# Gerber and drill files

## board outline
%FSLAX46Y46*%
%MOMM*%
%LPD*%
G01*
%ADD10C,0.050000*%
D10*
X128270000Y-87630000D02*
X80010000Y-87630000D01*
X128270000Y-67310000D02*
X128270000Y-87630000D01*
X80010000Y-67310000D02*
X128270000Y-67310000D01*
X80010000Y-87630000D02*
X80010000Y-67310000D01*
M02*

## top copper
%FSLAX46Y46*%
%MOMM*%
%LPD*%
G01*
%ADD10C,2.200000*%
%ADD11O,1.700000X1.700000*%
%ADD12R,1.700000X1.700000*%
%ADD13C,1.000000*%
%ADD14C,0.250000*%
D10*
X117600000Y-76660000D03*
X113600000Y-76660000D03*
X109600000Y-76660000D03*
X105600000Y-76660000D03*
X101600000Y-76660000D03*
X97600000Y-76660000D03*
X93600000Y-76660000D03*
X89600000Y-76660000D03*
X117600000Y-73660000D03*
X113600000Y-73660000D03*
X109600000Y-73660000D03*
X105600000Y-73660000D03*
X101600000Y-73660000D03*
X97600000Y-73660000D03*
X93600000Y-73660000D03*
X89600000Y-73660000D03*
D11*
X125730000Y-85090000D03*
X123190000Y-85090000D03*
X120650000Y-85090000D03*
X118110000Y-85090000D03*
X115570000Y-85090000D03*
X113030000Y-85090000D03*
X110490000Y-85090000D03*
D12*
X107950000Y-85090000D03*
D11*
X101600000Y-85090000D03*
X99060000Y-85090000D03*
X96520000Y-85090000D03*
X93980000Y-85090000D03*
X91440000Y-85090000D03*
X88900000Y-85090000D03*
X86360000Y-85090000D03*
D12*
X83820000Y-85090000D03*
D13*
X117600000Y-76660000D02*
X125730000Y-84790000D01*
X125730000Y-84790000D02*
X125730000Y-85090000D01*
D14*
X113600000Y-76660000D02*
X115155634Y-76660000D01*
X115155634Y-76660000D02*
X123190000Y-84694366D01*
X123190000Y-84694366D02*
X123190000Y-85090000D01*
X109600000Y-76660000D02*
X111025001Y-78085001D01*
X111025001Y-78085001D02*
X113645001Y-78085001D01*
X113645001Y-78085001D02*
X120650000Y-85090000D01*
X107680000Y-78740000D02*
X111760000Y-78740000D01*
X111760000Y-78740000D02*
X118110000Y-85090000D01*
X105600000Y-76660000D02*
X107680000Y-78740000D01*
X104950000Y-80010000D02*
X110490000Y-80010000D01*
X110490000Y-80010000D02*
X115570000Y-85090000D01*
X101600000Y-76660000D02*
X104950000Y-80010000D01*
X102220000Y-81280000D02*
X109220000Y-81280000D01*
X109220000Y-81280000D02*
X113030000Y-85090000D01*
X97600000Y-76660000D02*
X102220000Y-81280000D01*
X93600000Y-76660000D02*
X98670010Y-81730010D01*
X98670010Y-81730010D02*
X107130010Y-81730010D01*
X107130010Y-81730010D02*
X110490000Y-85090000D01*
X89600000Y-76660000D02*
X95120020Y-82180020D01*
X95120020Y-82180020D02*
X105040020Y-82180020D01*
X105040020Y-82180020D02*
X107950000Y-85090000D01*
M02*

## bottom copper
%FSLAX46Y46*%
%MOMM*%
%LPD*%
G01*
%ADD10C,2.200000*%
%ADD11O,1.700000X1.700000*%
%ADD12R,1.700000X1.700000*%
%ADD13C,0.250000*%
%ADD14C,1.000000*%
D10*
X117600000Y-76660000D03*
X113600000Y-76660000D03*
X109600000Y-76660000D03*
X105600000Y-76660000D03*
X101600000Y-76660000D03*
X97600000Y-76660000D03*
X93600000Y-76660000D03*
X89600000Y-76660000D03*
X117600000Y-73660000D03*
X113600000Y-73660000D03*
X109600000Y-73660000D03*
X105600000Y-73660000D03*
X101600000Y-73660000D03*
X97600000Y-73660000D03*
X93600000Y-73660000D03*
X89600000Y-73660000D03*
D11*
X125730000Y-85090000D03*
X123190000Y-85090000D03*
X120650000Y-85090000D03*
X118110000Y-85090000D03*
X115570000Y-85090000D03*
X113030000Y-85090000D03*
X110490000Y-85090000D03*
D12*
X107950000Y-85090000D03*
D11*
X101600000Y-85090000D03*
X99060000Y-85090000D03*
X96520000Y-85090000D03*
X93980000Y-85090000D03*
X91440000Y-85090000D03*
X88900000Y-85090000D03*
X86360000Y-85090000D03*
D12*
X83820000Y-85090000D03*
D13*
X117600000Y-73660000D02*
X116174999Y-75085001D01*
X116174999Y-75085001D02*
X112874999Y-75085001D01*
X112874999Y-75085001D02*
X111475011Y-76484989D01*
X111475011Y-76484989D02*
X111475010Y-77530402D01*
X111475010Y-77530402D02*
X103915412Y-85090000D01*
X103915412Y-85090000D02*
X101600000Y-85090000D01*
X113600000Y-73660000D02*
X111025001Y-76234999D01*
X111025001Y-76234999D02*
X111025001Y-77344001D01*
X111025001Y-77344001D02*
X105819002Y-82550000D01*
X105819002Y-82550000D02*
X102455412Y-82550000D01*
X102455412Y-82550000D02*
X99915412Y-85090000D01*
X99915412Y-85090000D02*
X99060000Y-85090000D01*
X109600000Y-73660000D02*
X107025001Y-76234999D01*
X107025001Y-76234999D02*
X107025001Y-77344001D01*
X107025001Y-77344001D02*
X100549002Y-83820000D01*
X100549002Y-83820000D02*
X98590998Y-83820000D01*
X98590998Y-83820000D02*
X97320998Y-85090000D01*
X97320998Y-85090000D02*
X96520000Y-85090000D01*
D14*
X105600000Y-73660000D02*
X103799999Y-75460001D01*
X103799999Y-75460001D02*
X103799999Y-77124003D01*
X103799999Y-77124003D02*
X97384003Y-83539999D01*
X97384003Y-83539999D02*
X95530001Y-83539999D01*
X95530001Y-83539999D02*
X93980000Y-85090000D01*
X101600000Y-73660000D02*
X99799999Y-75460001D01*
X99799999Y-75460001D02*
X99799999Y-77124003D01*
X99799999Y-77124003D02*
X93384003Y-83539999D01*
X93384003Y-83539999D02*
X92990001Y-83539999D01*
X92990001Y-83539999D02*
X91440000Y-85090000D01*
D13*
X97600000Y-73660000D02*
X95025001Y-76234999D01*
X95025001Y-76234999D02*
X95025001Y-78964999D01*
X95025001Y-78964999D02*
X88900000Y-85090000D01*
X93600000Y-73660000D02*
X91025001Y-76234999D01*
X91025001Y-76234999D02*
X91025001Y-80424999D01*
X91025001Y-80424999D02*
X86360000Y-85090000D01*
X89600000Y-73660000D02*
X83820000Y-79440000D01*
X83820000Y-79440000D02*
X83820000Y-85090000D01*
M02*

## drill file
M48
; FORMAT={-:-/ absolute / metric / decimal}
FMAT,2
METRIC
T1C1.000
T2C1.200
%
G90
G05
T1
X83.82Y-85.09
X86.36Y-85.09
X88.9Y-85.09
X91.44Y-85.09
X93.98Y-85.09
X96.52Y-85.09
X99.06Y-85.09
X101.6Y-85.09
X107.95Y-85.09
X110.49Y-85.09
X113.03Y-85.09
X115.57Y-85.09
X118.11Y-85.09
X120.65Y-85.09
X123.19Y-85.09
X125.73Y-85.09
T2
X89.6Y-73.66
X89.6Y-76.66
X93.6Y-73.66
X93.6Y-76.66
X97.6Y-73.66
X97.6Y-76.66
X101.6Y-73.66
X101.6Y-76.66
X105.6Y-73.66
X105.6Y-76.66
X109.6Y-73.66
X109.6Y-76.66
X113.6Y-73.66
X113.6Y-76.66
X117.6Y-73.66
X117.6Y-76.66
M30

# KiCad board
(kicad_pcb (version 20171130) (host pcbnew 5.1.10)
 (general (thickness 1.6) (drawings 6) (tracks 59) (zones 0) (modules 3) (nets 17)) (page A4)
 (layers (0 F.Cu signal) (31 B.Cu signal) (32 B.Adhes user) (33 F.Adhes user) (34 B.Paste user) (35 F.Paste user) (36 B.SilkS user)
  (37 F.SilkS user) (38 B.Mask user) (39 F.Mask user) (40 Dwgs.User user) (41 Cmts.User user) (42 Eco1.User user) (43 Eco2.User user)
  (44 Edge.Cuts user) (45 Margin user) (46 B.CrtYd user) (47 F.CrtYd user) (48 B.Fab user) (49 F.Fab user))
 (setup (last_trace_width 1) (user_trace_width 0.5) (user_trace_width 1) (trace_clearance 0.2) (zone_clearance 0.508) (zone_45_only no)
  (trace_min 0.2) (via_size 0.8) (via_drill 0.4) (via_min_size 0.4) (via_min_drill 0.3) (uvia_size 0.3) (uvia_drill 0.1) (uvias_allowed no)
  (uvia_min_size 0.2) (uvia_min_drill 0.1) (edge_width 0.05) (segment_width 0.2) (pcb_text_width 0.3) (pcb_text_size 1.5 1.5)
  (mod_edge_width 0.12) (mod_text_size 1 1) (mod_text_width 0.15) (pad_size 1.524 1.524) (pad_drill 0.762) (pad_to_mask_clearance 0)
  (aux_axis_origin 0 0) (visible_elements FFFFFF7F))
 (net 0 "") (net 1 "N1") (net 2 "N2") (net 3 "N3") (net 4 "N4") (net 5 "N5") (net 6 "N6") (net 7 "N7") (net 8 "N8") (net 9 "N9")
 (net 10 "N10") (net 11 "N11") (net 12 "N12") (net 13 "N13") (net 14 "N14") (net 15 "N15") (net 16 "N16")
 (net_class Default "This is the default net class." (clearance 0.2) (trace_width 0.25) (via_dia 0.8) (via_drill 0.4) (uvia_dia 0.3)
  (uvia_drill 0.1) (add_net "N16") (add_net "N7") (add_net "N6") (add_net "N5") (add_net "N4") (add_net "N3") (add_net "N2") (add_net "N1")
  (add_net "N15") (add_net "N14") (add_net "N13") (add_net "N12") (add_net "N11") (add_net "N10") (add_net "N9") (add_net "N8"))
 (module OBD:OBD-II (layer F.Cu) (at 105.6 72.66)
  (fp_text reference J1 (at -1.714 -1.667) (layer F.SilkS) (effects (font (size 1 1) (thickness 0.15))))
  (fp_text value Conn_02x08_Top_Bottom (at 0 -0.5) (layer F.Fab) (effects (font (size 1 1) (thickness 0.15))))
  (pad 16 thru_hole circle (at 12 4) (size 2.2 2.2) (drill 1.2) (layers *.Cu *.Mask) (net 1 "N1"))
  (pad 15 thru_hole circle (at 8 4) (size 2.2 2.2) (drill 1.2) (layers *.Cu *.Mask) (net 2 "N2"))
  (pad 14 thru_hole circle (at 4 4) (size 2.2 2.2) (drill 1.2) (layers *.Cu *.Mask) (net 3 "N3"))
  (pad 13 thru_hole circle (at 0 4) (size 2.2 2.2) (drill 1.2) (layers *.Cu *.Mask) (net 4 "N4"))
  (pad 12 thru_hole circle (at -4 4) (size 2.2 2.2) (drill 1.2) (layers *.Cu *.Mask) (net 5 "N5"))
  (pad 11 thru_hole circle (at -8 4) (size 2.2 2.2) (drill 1.2) (layers *.Cu *.Mask) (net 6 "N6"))
  (pad 10 thru_hole circle (at -12 4) (size 2.2 2.2) (drill 1.2) (layers *.Cu *.Mask) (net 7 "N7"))
  (pad 9 thru_hole circle (at -16 4) (size 2.2 2.2) (drill 1.2) (layers *.Cu *.Mask) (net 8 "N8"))
  (pad 8 thru_hole circle (at 12 1) (size 2.2 2.2) (drill 1.2) (layers *.Cu *.Mask) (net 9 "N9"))
  (pad 7 thru_hole circle (at 8 1) (size 2.2 2.2) (drill 1.2) (layers *.Cu *.Mask) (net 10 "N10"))
  (pad 6 thru_hole circle (at 4 1) (size 2.2 2.2) (drill 1.2) (layers *.Cu *.Mask) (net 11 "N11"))
  (pad 5 thru_hole circle (at 0 1) (size 2.2 2.2) (drill 1.2) (layers *.Cu *.Mask) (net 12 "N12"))
  (pad 4 thru_hole circle (at -4 1) (size 2.2 2.2) (drill 1.2) (layers *.Cu *.Mask) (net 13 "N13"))
  (pad 3 thru_hole circle (at -8 1) (size 2.2 2.2) (drill 1.2) (layers *.Cu *.Mask) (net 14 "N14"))
  (pad 2 thru_hole circle (at -12 1) (size 2.2 2.2) (drill 1.2) (layers *.Cu *.Mask) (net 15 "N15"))
  (pad 1 thru_hole circle (at -16 1) (size 2.2 2.2) (drill 1.2) (layers *.Cu *.Mask) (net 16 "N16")))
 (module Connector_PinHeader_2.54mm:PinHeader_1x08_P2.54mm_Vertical (layer F.Cu) (at 107.95 85.09 90)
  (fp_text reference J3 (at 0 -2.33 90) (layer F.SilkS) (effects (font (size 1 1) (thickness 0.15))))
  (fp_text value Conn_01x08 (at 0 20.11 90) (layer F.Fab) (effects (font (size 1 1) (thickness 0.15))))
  (pad 8 thru_hole oval (at 0 17.78 90) (size 1.7 1.7) (drill 1) (layers *.Cu *.Mask) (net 1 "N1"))
  (pad 7 thru_hole oval (at 0 15.24 90) (size 1.7 1.7) (drill 1) (layers *.Cu *.Mask) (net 2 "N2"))
  (pad 6 thru_hole oval (at 0 12.7 90) (size 1.7 1.7) (drill 1) (layers *.Cu *.Mask) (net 3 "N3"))
  (pad 5 thru_hole oval (at 0 10.16 90) (size 1.7 1.7) (drill 1) (layers *.Cu *.Mask) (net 4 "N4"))
  (pad 4 thru_hole oval (at 0 7.62 90) (size 1.7 1.7) (drill 1) (layers *.Cu *.Mask) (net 5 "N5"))
  (pad 3 thru_hole oval (at 0 5.08 90) (size 1.7 1.7) (drill 1) (layers *.Cu *.Mask) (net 6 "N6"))
  (pad 2 thru_hole oval (at 0 2.54 90) (size 1.7 1.7) (drill 1) (layers *.Cu *.Mask) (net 7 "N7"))
  (pad 1 thru_hole rect (at 0 0 90) (size 1.7 1.7) (drill 1) (layers *.Cu *.Mask) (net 8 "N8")))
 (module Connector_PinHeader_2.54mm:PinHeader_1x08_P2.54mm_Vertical (layer F.Cu) (at 83.82 85.09 90)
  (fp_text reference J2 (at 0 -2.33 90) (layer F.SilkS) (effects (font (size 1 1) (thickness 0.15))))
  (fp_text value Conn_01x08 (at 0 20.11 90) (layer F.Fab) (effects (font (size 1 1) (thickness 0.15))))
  (pad 8 thru_hole oval (at 0 17.78 90) (size 1.7 1.7) (drill 1) (layers *.Cu *.Mask) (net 9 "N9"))
  (pad 7 thru_hole oval (at 0 15.24 90) (size 1.7 1.7) (drill 1) (layers *.Cu *.Mask) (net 10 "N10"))
  (pad 6 thru_hole oval (at 0 12.7 90) (size 1.7 1.7) (drill 1) (layers *.Cu *.Mask) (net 11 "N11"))
  (pad 5 thru_hole oval (at 0 10.16 90) (size 1.7 1.7) (drill 1) (layers *.Cu *.Mask) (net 12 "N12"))
  (pad 4 thru_hole oval (at 0 7.62 90) (size 1.7 1.7) (drill 1) (layers *.Cu *.Mask) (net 13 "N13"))
  (pad 3 thru_hole oval (at 0 5.08 90) (size 1.7 1.7) (drill 1) (layers *.Cu *.Mask) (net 14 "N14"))
  (pad 2 thru_hole oval (at 0 2.54 90) (size 1.7 1.7) (drill 1) (layers *.Cu *.Mask) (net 15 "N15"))
  (pad 1 thru_hole rect (at 0 0 90) (size 1.7 1.7) (drill 1) (layers *.Cu *.Mask) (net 16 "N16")))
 (gr_line (start 128.27 87.63) (end 80.01 87.63) (layer Edge.Cuts) (width 0.05))
 (gr_line (start 128.27 67.31) (end 128.27 87.63) (layer Edge.Cuts) (width 0.05))
 (gr_line (start 80.01 67.31) (end 128.27 67.31) (layer Edge.Cuts) (width 0.05))
 (gr_line (start 80.01 87.63) (end 80.01 67.31) (layer Edge.Cuts) (width 0.05))
 (segment (start 117.6 76.66) (end 125.73 84.79) (width 1) (layer F.Cu) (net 1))
 (segment (start 125.73 84.79) (end 125.73 85.09) (width 1) (layer F.Cu) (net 1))
 (segment (start 113.6 76.66) (end 115.155634 76.66) (width 0.25) (layer F.Cu) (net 2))
 (segment (start 115.155634 76.66) (end 123.19 84.694366) (width 0.25) (layer F.Cu) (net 2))
 (segment (start 123.19 84.694366) (end 123.19 85.09) (width 0.25) (layer F.Cu) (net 2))
 (segment (start 109.6 76.66) (end 111.025001 78.085001) (width 0.25) (layer F.Cu) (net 3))
 (segment (start 111.025001 78.085001) (end 113.645001 78.085001) (width 0.25) (layer F.Cu) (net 3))
 (segment (start 113.645001 78.085001) (end 120.65 85.09) (width 0.25) (layer F.Cu) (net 3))
 (segment (start 107.68 78.74) (end 111.76 78.74) (width 0.25) (layer F.Cu) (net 4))
 (segment (start 111.76 78.74) (end 118.11 85.09) (width 0.25) (layer F.Cu) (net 4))
 (segment (start 105.6 76.66) (end 107.68 78.74) (width 0.25) (layer F.Cu) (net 4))
 (segment (start 104.95 80.01) (end 110.49 80.01) (width 0.25) (layer F.Cu) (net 5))
 (segment (start 110.49 80.01) (end 115.57 85.09) (width 0.25) (layer F.Cu) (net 5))
 (segment (start 101.6 76.66) (end 104.95 80.01) (width 0.25) (layer F.Cu) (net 5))
 (segment (start 102.22 81.28) (end 109.22 81.28) (width 0.25) (layer F.Cu) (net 6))
 (segment (start 109.22 81.28) (end 113.03 85.09) (width 0.25) (layer F.Cu) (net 6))
 (segment (start 97.6 76.66) (end 102.22 81.28) (width 0.25) (layer F.Cu) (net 6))
 (segment (start 93.6 76.66) (end 98.67001 81.73001) (width 0.25) (layer F.Cu) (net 7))
 (segment (start 98.67001 81.73001) (end 107.13001 81.73001) (width 0.25) (layer F.Cu) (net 7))
 (segment (start 107.13001 81.73001) (end 110.49 85.09) (width 0.25) (layer F.Cu) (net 7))
 (segment (start 89.6 76.66) (end 95.12002 82.18002) (width 0.25) (layer F.Cu) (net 8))
 (segment (start 95.12002 82.18002) (end 105.04002 82.18002) (width 0.25) (layer F.Cu) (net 8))
 (segment (start 105.04002 82.18002) (end 107.95 85.09) (width 0.25) (layer F.Cu) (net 8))
 (segment (start 117.6 73.66) (end 116.174999 75.085001) (width 0.25) (layer B.Cu) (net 9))
 (segment (start 116.174999 75.085001) (end 112.874999 75.085001) (width 0.25) (layer B.Cu) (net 9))
 (segment (start 112.874999 75.085001) (end 111.475011 76.484989) (width 0.25) (layer B.Cu) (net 9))
 (segment (start 111.475011 76.484989) (end 111.47501 77.530402) (width 0.25) (layer B.Cu) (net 9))
 (segment (start 111.47501 77.530402) (end 103.915412 85.09) (width 0.25) (layer B.Cu) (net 9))
 (segment (start 103.915412 85.09) (end 101.6 85.09) (width 0.25) (layer B.Cu) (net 9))
 (segment (start 113.6 73.66) (end 111.025001 76.234999) (width 0.25) (layer B.Cu) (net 10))
 (segment (start 111.025001 76.234999) (end 111.025001 77.344001) (width 0.25) (layer B.Cu) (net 10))
 (segment (start 111.025001 77.344001) (end 105.819002 82.55) (width 0.25) (layer B.Cu) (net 10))
 (segment (start 105.819002 82.55) (end 102.455412 82.55) (width 0.25) (layer B.Cu) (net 10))
 (segment (start 102.455412 82.55) (end 99.915412 85.09) (width 0.25) (layer B.Cu) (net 10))
 (segment (start 99.915412 85.09) (end 99.06 85.09) (width 0.25) (layer B.Cu) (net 10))
 (segment (start 109.6 73.66) (end 107.025001 76.234999) (width 0.25) (layer B.Cu) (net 11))
 (segment (start 107.025001 76.234999) (end 107.025001 77.344001) (width 0.25) (layer B.Cu) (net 11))
 (segment (start 107.025001 77.344001) (end 100.549002 83.82) (width 0.25) (layer B.Cu) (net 11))
 (segment (start 100.549002 83.82) (end 98.590998 83.82) (width 0.25) (layer B.Cu) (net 11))
 (segment (start 98.590998 83.82) (end 97.320998 85.09) (width 0.25) (layer B.Cu) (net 11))
 (segment (start 97.320998 85.09) (end 96.52 85.09) (width 0.25) (layer B.Cu) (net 11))
 (segment (start 105.6 73.66) (end 103.799999 75.460001) (width 1) (layer B.Cu) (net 12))
 (segment (start 103.799999 75.460001) (end 103.799999 77.124003) (width 1) (layer B.Cu) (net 12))
 (segment (start 103.799999 77.124003) (end 97.384003 83.539999) (width 1) (layer B.Cu) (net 12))
 (segment (start 97.384003 83.539999) (end 95.530001 83.539999) (width 1) (layer B.Cu) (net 12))
 (segment (start 95.530001 83.539999) (end 93.98 85.09) (width 1) (layer B.Cu) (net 12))
 (segment (start 101.6 73.66) (end 99.799999 75.460001) (width 1) (layer B.Cu) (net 13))
 (segment (start 99.799999 75.460001) (end 99.799999 77.124003) (width 1) (layer B.Cu) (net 13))
 (segment (start 99.799999 77.124003) (end 93.384003 83.539999) (width 1) (layer B.Cu) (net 13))
 (segment (start 93.384003 83.539999) (end 92.990001 83.539999) (width 1) (layer B.Cu) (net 13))
 (segment (start 92.990001 83.539999) (end 91.44 85.09) (width 1) (layer B.Cu) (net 13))
 (segment (start 97.6 73.66) (end 95.025001 76.234999) (width 0.25) (layer B.Cu) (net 14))
 (segment (start 95.025001 76.234999) (end 95.025001 78.964999) (width 0.25) (layer B.Cu) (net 14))
 (segment (start 95.025001 78.964999) (end 88.9 85.09) (width 0.25) (layer B.Cu) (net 14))
 (segment (start 93.6 73.66) (end 91.025001 76.234999) (width 0.25) (layer B.Cu) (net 15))
 (segment (start 91.025001 76.234999) (end 91.025001 80.424999) (width 0.25) (layer B.Cu) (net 15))
 (segment (start 91.025001 80.424999) (end 86.36 85.09) (width 0.25) (layer B.Cu) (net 15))
 (segment (start 89.6 73.66) (end 83.82 79.44) (width 0.25) (layer B.Cu) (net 16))
 (segment (start 83.82 79.44) (end 83.82 85.09) (width 0.25) (layer B.Cu) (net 16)))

